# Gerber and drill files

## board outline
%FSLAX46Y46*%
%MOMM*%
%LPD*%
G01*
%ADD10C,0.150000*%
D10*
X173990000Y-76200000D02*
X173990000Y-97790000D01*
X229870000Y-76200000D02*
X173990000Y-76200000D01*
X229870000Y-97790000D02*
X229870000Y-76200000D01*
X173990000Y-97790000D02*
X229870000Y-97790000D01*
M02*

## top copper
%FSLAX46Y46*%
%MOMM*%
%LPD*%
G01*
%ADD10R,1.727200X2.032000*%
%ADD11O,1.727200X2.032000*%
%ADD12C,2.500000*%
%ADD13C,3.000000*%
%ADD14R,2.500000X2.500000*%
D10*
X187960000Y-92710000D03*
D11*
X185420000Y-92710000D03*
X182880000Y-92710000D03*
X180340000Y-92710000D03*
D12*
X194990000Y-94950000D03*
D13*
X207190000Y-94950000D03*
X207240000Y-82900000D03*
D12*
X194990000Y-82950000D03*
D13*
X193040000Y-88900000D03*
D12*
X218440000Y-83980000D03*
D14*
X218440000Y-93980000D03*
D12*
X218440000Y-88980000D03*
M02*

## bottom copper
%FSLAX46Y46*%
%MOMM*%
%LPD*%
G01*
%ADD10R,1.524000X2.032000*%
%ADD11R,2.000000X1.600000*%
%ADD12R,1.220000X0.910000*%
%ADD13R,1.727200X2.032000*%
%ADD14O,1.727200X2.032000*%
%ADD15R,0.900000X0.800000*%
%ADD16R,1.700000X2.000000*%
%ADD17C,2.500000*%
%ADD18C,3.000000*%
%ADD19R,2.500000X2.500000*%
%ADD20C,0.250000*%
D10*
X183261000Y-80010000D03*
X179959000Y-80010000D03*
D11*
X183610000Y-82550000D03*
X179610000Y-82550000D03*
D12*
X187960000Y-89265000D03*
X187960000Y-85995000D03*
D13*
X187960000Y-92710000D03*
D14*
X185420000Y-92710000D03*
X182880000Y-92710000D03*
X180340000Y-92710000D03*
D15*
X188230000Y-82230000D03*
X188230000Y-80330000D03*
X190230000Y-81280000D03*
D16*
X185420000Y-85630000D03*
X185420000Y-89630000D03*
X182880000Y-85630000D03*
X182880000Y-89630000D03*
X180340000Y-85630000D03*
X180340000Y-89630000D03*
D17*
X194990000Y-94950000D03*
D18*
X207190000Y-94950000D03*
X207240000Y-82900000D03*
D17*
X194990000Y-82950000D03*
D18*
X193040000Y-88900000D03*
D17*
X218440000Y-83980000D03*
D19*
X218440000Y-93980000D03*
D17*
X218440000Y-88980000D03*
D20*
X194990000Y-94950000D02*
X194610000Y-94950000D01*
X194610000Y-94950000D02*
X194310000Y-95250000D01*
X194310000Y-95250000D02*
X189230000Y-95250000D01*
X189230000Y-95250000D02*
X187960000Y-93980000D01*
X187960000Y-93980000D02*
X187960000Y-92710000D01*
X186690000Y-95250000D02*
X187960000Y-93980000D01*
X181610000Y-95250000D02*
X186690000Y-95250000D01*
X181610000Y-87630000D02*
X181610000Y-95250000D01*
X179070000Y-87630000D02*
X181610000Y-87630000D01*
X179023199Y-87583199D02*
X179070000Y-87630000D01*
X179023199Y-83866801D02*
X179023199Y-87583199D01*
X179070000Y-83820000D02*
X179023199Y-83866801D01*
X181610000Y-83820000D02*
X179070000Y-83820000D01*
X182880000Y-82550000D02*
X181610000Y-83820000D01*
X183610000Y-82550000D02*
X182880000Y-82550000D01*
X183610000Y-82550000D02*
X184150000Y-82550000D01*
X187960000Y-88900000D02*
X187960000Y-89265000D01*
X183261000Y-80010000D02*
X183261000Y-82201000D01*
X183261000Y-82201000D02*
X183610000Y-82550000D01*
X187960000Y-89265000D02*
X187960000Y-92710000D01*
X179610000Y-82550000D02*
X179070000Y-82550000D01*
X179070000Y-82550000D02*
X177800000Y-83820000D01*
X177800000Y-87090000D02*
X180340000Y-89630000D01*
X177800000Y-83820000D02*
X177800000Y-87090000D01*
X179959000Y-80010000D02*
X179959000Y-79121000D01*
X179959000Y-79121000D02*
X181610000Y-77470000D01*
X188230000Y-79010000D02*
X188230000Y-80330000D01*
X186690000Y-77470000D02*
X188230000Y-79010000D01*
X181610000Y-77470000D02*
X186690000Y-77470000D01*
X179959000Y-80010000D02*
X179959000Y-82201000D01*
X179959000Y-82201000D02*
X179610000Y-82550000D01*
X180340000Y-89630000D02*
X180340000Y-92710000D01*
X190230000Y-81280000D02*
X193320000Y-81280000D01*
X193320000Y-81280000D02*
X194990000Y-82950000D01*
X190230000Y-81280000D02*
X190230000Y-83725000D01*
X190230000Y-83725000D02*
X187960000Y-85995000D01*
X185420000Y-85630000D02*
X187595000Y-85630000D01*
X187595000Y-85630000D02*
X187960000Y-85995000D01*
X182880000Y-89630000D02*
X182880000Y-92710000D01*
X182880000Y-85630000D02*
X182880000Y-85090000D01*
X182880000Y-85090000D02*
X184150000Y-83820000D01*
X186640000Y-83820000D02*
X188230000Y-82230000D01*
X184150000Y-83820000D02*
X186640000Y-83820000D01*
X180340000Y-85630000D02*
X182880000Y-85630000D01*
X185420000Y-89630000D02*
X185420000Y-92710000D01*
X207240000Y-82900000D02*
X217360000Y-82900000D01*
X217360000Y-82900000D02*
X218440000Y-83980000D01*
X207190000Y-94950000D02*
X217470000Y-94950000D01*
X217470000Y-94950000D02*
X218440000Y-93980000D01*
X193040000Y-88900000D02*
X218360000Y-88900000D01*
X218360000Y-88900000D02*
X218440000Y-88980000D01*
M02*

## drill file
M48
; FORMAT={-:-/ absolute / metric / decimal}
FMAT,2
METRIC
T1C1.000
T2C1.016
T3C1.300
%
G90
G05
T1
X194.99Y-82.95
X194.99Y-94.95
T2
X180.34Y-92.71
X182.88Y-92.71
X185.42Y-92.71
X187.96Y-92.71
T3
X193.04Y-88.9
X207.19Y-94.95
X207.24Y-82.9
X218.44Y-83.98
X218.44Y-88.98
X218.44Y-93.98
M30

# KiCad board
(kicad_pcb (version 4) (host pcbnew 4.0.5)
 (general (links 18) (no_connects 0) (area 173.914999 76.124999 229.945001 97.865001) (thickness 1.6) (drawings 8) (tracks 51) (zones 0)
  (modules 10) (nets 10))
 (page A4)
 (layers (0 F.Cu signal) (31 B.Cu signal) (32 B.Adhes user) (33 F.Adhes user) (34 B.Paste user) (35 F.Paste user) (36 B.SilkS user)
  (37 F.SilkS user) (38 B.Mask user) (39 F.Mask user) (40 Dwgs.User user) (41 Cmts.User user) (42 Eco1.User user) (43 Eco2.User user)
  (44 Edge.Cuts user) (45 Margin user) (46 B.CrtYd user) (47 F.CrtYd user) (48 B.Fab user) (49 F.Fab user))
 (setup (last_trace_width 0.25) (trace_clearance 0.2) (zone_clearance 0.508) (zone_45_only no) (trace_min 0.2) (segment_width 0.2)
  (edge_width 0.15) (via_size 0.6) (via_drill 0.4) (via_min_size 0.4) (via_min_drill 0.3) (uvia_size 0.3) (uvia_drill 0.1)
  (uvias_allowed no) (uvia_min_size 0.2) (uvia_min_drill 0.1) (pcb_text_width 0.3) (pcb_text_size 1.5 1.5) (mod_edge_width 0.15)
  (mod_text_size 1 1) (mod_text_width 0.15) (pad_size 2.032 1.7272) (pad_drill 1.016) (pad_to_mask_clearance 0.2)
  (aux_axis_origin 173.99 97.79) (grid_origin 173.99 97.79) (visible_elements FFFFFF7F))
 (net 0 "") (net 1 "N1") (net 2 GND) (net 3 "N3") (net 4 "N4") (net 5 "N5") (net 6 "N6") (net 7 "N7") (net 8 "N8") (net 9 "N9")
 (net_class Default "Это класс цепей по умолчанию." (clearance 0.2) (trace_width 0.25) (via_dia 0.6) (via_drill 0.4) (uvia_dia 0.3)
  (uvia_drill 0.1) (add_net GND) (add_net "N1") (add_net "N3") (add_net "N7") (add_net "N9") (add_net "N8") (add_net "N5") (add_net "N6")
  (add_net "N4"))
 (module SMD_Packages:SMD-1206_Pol (layer B.Cu) (at 181.61 80.01 180)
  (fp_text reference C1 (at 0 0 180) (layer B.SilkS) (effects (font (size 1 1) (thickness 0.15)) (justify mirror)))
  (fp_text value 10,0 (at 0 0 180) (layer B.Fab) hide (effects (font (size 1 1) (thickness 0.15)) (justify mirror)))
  (pad 1 smd rect (at -1.651 0 180) (size 1.524 2.032) (layers B.Cu B.Paste B.Mask) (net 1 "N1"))
  (pad 2 smd rect (at 1.651 0 180) (size 1.524 2.032) (layers B.Cu B.Paste B.Mask) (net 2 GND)))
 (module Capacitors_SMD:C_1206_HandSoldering (layer B.Cu) (at 181.61 82.55 180)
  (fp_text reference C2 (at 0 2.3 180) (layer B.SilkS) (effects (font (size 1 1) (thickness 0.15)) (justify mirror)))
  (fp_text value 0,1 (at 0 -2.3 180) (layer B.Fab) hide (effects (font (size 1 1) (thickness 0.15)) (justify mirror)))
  (pad 1 smd rect (at -2 0 180) (size 2 1.6) (layers B.Cu B.Paste B.Mask) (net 1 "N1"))
  (pad 2 smd rect (at 2 0 180) (size 2 1.6) (layers B.Cu B.Paste B.Mask) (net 2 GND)))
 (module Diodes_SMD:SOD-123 (layer B.Cu) (at 187.96 87.63 90)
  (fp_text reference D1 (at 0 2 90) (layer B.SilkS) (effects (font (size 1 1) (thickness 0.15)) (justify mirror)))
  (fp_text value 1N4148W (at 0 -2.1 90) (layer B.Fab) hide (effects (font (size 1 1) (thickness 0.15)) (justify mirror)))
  (pad 1 smd rect (at -1.635 0 90) (size 0.91 1.22) (layers B.Cu B.Paste B.Mask) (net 1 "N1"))
  (pad 2 smd rect (at 1.635 0 90) (size 0.91 1.22) (layers B.Cu B.Paste B.Mask) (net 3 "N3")))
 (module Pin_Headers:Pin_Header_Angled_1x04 (layer F.Cu) (at 187.96 92.71 270)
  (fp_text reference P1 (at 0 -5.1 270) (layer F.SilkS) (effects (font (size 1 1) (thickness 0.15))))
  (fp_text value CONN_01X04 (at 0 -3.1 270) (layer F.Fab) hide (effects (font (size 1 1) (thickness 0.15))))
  (pad 1 thru_hole rect (at 0 0 270) (size 2.032 1.7272) (drill 1.016) (layers *.Cu *.Mask) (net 1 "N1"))
  (pad 2 thru_hole oval (at 0 2.54 270) (size 2.032 1.7272) (drill 1.016) (layers *.Cu *.Mask) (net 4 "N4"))
  (pad 3 thru_hole oval (at 0 5.08 270) (size 2.032 1.7272) (drill 1.016) (layers *.Cu *.Mask) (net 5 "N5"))
  (pad 4 thru_hole oval (at 0 7.62 270) (size 2.032 1.7272) (drill 1.016) (layers *.Cu *.Mask) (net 2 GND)))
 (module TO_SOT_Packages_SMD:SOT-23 (layer B.Cu) (at 189.23 81.28)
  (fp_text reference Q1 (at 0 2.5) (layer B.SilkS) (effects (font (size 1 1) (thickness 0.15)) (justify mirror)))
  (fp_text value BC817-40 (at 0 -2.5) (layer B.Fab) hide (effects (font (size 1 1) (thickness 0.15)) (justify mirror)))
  (pad 1 smd rect (at -1 0.95) (size 0.9 0.8) (layers B.Cu B.Paste B.Mask) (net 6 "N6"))
  (pad 2 smd rect (at -1 -0.95) (size 0.9 0.8) (layers B.Cu B.Paste B.Mask) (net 2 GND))
  (pad 3 smd rect (at 1 0) (size 0.9 0.8) (layers B.Cu B.Paste B.Mask) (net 3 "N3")))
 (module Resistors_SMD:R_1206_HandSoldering (layer B.Cu) (at 185.42 87.63 270)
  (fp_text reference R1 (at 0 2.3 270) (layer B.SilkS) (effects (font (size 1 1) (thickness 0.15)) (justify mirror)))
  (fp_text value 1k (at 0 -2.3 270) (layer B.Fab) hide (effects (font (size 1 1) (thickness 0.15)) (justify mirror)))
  (pad 1 smd rect (at -2 0 270) (size 2 1.7) (layers B.Cu B.Paste B.Mask) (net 3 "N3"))
  (pad 2 smd rect (at 2 0 270) (size 2 1.7) (layers B.Cu B.Paste B.Mask) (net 4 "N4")))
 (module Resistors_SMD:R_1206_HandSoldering (layer B.Cu) (at 182.88 87.63 270)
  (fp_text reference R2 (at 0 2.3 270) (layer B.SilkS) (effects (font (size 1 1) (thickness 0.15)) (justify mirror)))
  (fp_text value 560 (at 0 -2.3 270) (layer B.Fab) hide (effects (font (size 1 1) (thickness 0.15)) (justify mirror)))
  (pad 1 smd rect (at -2 0 270) (size 2 1.7) (layers B.Cu B.Paste B.Mask) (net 6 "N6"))
  (pad 2 smd rect (at 2 0 270) (size 2 1.7) (layers B.Cu B.Paste B.Mask) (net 5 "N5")))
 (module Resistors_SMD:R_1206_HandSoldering (layer B.Cu) (at 180.34 87.63 270)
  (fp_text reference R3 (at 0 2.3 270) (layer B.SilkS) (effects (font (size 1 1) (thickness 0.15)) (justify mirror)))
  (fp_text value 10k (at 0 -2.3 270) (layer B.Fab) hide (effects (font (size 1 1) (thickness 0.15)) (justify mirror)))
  (pad 1 smd rect (at -2 0 270) (size 2 1.7) (layers B.Cu B.Paste B.Mask) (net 6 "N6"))
  (pad 2 smd rect (at 2 0 270) (size 2 1.7) (layers B.Cu B.Paste B.Mask) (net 2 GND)))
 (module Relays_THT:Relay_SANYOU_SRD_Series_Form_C (layer F.Cu) (at 193.04 88.9)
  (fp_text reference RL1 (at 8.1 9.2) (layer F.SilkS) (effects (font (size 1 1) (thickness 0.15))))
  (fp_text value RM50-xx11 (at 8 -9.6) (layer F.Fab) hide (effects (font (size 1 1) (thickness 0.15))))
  (pad 2 thru_hole circle (at 1.95 6.05 90) (size 2.5 2.5) (drill 1) (layers *.Cu *.Mask) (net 1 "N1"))
  (pad 3 thru_hole circle (at 14.15 6.05 90) (size 3 3) (drill 1.3) (layers *.Cu *.Mask) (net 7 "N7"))
  (pad 4 thru_hole circle (at 14.2 -6 90) (size 3 3) (drill 1.3) (layers *.Cu *.Mask) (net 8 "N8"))
  (pad 5 thru_hole circle (at 1.95 -5.95 90) (size 2.5 2.5) (drill 1) (layers *.Cu *.Mask) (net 3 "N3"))
  (pad 1 thru_hole circle (at 0 0 90) (size 3 3) (drill 1.3) (layers *.Cu *.Mask) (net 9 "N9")))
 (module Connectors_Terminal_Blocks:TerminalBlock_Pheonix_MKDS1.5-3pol (layer F.Cu) (at 218.44 93.98 90)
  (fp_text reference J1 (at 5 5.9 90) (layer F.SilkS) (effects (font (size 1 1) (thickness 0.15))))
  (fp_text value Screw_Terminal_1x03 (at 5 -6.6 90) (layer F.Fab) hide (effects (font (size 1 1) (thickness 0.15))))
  (pad 3 thru_hole circle (at 10 0 90) (size 2.5 2.5) (drill 1.3) (layers *.Cu *.Mask) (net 8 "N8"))
  (pad 1 thru_hole rect (at 0 0 90) (size 2.5 2.5) (drill 1.3) (layers *.Cu *.Mask) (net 7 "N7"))
  (pad 2 thru_hole circle (at 5 0 90) (size 2.5 2.5) (drill 1.3) (layers *.Cu *.Mask) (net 9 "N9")))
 (gr_line (start 173.99 76.2) (end 173.99 97.79) (angle 90) (layer Edge.Cuts) (width 0.15))
 (gr_line (start 229.87 76.2) (end 173.99 76.2) (angle 90) (layer Edge.Cuts) (width 0.15))
 (gr_line (start 229.87 97.79) (end 229.87 76.2) (angle 90) (layer Edge.Cuts) (width 0.15))
 (gr_line (start 173.99 97.79) (end 229.87 97.79) (angle 90) (layer Edge.Cuts) (width 0.15))
 (segment (start 194.99 94.95) (end 194.61 94.95) (width 0.25) (layer B.Cu) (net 1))
 (segment (start 194.61 94.95) (end 194.31 95.25) (width 0.25) (layer B.Cu) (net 1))
 (segment (start 194.31 95.25) (end 189.23 95.25) (width 0.25) (layer B.Cu) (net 1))
 (segment (start 189.23 95.25) (end 187.96 93.98) (width 0.25) (layer B.Cu) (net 1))
 (segment (start 187.96 93.98) (end 187.96 92.71) (width 0.25) (layer B.Cu) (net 1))
 (segment (start 186.69 95.25) (end 187.96 93.98) (width 0.25) (layer B.Cu) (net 1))
 (segment (start 181.61 95.25) (end 186.69 95.25) (width 0.25) (layer B.Cu) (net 1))
 (segment (start 181.61 87.63) (end 181.61 95.25) (width 0.25) (layer B.Cu) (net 1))
 (segment (start 179.07 87.63) (end 181.61 87.63) (width 0.25) (layer B.Cu) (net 1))
 (segment (start 179.023199 87.583199) (end 179.07 87.63) (width 0.25) (layer B.Cu) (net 1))
 (segment (start 179.023199 83.866801) (end 179.023199 87.583199) (width 0.25) (layer B.Cu) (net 1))
 (segment (start 179.07 83.82) (end 179.023199 83.866801) (width 0.25) (layer B.Cu) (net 1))
 (segment (start 181.61 83.82) (end 179.07 83.82) (width 0.25) (layer B.Cu) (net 1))
 (segment (start 182.88 82.55) (end 181.61 83.82) (width 0.25) (layer B.Cu) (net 1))
 (segment (start 183.61 82.55) (end 182.88 82.55) (width 0.25) (layer B.Cu) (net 1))
 (segment (start 183.61 82.55) (end 184.15 82.55) (width 0.25) (layer B.Cu) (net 1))
 (segment (start 187.96 88.9) (end 187.96 89.265) (width 0.25) (layer B.Cu) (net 1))
 (segment (start 183.261 80.01) (end 183.261 82.201) (width 0.25) (layer B.Cu) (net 1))
 (segment (start 183.261 82.201) (end 183.61 82.55) (width 0.25) (layer B.Cu) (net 1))
 (segment (start 187.96 89.265) (end 187.96 92.71) (width 0.25) (layer B.Cu) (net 1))
 (segment (start 179.61 82.55) (end 179.07 82.55) (width 0.25) (layer B.Cu) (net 2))
 (segment (start 179.07 82.55) (end 177.8 83.82) (width 0.25) (layer B.Cu) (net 2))
 (segment (start 177.8 87.09) (end 180.34 89.63) (width 0.25) (layer B.Cu) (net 2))
 (segment (start 177.8 83.82) (end 177.8 87.09) (width 0.25) (layer B.Cu) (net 2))
 (segment (start 179.959 80.01) (end 179.959 79.121) (width 0.25) (layer B.Cu) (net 2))
 (segment (start 179.959 79.121) (end 181.61 77.47) (width 0.25) (layer B.Cu) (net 2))
 (segment (start 188.23 79.01) (end 188.23 80.33) (width 0.25) (layer B.Cu) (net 2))
 (segment (start 186.69 77.47) (end 188.23 79.01) (width 0.25) (layer B.Cu) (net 2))
 (segment (start 181.61 77.47) (end 186.69 77.47) (width 0.25) (layer B.Cu) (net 2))
 (segment (start 179.959 80.01) (end 179.959 82.201) (width 0.25) (layer B.Cu) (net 2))
 (segment (start 179.959 82.201) (end 179.61 82.55) (width 0.25) (layer B.Cu) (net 2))
 (segment (start 180.34 89.63) (end 180.34 92.71) (width 0.25) (layer B.Cu) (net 2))
 (segment (start 190.23 81.28) (end 193.32 81.28) (width 0.25) (layer B.Cu) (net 3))
 (segment (start 193.32 81.28) (end 194.99 82.95) (width 0.25) (layer B.Cu) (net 3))
 (segment (start 190.23 81.28) (end 190.23 83.725) (width 0.25) (layer B.Cu) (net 3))
 (segment (start 190.23 83.725) (end 187.96 85.995) (width 0.25) (layer B.Cu) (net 3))
 (segment (start 185.42 85.63) (end 187.595 85.63) (width 0.25) (layer B.Cu) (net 3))
 (segment (start 187.595 85.63) (end 187.96 85.995) (width 0.25) (layer B.Cu) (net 3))
 (segment (start 182.88 89.63) (end 182.88 92.71) (width 0.25) (layer B.Cu) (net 5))
 (segment (start 182.88 85.63) (end 182.88 85.09) (width 0.25) (layer B.Cu) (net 6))
 (segment (start 182.88 85.09) (end 184.15 83.82) (width 0.25) (layer B.Cu) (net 6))
 (segment (start 186.64 83.82) (end 188.23 82.23) (width 0.25) (layer B.Cu) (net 6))
 (segment (start 184.15 83.82) (end 186.64 83.82) (width 0.25) (layer B.Cu) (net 6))
 (segment (start 180.34 85.63) (end 182.88 85.63) (width 0.25) (layer B.Cu) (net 6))
 (segment (start 185.42 89.63) (end 185.42 92.71) (width 0.25) (layer B.Cu) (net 4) (status C00000))
 (segment (start 207.24 82.9) (end 217.36 82.9) (width 0.25) (layer B.Cu) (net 8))
 (segment (start 217.36 82.9) (end 218.44 83.98) (width 0.25) (layer B.Cu) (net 8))
 (segment (start 207.19 94.95) (end 217.47 94.95) (width 0.25) (layer B.Cu) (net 7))
 (segment (start 217.47 94.95) (end 218.44 93.98) (width 0.25) (layer B.Cu) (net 7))
 (segment (start 193.04 88.9) (end 218.36 88.9) (width 0.25) (layer B.Cu) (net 9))
 (segment (start 218.36 88.9) (end 218.44 88.98) (width 0.25) (layer B.Cu) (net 9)))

